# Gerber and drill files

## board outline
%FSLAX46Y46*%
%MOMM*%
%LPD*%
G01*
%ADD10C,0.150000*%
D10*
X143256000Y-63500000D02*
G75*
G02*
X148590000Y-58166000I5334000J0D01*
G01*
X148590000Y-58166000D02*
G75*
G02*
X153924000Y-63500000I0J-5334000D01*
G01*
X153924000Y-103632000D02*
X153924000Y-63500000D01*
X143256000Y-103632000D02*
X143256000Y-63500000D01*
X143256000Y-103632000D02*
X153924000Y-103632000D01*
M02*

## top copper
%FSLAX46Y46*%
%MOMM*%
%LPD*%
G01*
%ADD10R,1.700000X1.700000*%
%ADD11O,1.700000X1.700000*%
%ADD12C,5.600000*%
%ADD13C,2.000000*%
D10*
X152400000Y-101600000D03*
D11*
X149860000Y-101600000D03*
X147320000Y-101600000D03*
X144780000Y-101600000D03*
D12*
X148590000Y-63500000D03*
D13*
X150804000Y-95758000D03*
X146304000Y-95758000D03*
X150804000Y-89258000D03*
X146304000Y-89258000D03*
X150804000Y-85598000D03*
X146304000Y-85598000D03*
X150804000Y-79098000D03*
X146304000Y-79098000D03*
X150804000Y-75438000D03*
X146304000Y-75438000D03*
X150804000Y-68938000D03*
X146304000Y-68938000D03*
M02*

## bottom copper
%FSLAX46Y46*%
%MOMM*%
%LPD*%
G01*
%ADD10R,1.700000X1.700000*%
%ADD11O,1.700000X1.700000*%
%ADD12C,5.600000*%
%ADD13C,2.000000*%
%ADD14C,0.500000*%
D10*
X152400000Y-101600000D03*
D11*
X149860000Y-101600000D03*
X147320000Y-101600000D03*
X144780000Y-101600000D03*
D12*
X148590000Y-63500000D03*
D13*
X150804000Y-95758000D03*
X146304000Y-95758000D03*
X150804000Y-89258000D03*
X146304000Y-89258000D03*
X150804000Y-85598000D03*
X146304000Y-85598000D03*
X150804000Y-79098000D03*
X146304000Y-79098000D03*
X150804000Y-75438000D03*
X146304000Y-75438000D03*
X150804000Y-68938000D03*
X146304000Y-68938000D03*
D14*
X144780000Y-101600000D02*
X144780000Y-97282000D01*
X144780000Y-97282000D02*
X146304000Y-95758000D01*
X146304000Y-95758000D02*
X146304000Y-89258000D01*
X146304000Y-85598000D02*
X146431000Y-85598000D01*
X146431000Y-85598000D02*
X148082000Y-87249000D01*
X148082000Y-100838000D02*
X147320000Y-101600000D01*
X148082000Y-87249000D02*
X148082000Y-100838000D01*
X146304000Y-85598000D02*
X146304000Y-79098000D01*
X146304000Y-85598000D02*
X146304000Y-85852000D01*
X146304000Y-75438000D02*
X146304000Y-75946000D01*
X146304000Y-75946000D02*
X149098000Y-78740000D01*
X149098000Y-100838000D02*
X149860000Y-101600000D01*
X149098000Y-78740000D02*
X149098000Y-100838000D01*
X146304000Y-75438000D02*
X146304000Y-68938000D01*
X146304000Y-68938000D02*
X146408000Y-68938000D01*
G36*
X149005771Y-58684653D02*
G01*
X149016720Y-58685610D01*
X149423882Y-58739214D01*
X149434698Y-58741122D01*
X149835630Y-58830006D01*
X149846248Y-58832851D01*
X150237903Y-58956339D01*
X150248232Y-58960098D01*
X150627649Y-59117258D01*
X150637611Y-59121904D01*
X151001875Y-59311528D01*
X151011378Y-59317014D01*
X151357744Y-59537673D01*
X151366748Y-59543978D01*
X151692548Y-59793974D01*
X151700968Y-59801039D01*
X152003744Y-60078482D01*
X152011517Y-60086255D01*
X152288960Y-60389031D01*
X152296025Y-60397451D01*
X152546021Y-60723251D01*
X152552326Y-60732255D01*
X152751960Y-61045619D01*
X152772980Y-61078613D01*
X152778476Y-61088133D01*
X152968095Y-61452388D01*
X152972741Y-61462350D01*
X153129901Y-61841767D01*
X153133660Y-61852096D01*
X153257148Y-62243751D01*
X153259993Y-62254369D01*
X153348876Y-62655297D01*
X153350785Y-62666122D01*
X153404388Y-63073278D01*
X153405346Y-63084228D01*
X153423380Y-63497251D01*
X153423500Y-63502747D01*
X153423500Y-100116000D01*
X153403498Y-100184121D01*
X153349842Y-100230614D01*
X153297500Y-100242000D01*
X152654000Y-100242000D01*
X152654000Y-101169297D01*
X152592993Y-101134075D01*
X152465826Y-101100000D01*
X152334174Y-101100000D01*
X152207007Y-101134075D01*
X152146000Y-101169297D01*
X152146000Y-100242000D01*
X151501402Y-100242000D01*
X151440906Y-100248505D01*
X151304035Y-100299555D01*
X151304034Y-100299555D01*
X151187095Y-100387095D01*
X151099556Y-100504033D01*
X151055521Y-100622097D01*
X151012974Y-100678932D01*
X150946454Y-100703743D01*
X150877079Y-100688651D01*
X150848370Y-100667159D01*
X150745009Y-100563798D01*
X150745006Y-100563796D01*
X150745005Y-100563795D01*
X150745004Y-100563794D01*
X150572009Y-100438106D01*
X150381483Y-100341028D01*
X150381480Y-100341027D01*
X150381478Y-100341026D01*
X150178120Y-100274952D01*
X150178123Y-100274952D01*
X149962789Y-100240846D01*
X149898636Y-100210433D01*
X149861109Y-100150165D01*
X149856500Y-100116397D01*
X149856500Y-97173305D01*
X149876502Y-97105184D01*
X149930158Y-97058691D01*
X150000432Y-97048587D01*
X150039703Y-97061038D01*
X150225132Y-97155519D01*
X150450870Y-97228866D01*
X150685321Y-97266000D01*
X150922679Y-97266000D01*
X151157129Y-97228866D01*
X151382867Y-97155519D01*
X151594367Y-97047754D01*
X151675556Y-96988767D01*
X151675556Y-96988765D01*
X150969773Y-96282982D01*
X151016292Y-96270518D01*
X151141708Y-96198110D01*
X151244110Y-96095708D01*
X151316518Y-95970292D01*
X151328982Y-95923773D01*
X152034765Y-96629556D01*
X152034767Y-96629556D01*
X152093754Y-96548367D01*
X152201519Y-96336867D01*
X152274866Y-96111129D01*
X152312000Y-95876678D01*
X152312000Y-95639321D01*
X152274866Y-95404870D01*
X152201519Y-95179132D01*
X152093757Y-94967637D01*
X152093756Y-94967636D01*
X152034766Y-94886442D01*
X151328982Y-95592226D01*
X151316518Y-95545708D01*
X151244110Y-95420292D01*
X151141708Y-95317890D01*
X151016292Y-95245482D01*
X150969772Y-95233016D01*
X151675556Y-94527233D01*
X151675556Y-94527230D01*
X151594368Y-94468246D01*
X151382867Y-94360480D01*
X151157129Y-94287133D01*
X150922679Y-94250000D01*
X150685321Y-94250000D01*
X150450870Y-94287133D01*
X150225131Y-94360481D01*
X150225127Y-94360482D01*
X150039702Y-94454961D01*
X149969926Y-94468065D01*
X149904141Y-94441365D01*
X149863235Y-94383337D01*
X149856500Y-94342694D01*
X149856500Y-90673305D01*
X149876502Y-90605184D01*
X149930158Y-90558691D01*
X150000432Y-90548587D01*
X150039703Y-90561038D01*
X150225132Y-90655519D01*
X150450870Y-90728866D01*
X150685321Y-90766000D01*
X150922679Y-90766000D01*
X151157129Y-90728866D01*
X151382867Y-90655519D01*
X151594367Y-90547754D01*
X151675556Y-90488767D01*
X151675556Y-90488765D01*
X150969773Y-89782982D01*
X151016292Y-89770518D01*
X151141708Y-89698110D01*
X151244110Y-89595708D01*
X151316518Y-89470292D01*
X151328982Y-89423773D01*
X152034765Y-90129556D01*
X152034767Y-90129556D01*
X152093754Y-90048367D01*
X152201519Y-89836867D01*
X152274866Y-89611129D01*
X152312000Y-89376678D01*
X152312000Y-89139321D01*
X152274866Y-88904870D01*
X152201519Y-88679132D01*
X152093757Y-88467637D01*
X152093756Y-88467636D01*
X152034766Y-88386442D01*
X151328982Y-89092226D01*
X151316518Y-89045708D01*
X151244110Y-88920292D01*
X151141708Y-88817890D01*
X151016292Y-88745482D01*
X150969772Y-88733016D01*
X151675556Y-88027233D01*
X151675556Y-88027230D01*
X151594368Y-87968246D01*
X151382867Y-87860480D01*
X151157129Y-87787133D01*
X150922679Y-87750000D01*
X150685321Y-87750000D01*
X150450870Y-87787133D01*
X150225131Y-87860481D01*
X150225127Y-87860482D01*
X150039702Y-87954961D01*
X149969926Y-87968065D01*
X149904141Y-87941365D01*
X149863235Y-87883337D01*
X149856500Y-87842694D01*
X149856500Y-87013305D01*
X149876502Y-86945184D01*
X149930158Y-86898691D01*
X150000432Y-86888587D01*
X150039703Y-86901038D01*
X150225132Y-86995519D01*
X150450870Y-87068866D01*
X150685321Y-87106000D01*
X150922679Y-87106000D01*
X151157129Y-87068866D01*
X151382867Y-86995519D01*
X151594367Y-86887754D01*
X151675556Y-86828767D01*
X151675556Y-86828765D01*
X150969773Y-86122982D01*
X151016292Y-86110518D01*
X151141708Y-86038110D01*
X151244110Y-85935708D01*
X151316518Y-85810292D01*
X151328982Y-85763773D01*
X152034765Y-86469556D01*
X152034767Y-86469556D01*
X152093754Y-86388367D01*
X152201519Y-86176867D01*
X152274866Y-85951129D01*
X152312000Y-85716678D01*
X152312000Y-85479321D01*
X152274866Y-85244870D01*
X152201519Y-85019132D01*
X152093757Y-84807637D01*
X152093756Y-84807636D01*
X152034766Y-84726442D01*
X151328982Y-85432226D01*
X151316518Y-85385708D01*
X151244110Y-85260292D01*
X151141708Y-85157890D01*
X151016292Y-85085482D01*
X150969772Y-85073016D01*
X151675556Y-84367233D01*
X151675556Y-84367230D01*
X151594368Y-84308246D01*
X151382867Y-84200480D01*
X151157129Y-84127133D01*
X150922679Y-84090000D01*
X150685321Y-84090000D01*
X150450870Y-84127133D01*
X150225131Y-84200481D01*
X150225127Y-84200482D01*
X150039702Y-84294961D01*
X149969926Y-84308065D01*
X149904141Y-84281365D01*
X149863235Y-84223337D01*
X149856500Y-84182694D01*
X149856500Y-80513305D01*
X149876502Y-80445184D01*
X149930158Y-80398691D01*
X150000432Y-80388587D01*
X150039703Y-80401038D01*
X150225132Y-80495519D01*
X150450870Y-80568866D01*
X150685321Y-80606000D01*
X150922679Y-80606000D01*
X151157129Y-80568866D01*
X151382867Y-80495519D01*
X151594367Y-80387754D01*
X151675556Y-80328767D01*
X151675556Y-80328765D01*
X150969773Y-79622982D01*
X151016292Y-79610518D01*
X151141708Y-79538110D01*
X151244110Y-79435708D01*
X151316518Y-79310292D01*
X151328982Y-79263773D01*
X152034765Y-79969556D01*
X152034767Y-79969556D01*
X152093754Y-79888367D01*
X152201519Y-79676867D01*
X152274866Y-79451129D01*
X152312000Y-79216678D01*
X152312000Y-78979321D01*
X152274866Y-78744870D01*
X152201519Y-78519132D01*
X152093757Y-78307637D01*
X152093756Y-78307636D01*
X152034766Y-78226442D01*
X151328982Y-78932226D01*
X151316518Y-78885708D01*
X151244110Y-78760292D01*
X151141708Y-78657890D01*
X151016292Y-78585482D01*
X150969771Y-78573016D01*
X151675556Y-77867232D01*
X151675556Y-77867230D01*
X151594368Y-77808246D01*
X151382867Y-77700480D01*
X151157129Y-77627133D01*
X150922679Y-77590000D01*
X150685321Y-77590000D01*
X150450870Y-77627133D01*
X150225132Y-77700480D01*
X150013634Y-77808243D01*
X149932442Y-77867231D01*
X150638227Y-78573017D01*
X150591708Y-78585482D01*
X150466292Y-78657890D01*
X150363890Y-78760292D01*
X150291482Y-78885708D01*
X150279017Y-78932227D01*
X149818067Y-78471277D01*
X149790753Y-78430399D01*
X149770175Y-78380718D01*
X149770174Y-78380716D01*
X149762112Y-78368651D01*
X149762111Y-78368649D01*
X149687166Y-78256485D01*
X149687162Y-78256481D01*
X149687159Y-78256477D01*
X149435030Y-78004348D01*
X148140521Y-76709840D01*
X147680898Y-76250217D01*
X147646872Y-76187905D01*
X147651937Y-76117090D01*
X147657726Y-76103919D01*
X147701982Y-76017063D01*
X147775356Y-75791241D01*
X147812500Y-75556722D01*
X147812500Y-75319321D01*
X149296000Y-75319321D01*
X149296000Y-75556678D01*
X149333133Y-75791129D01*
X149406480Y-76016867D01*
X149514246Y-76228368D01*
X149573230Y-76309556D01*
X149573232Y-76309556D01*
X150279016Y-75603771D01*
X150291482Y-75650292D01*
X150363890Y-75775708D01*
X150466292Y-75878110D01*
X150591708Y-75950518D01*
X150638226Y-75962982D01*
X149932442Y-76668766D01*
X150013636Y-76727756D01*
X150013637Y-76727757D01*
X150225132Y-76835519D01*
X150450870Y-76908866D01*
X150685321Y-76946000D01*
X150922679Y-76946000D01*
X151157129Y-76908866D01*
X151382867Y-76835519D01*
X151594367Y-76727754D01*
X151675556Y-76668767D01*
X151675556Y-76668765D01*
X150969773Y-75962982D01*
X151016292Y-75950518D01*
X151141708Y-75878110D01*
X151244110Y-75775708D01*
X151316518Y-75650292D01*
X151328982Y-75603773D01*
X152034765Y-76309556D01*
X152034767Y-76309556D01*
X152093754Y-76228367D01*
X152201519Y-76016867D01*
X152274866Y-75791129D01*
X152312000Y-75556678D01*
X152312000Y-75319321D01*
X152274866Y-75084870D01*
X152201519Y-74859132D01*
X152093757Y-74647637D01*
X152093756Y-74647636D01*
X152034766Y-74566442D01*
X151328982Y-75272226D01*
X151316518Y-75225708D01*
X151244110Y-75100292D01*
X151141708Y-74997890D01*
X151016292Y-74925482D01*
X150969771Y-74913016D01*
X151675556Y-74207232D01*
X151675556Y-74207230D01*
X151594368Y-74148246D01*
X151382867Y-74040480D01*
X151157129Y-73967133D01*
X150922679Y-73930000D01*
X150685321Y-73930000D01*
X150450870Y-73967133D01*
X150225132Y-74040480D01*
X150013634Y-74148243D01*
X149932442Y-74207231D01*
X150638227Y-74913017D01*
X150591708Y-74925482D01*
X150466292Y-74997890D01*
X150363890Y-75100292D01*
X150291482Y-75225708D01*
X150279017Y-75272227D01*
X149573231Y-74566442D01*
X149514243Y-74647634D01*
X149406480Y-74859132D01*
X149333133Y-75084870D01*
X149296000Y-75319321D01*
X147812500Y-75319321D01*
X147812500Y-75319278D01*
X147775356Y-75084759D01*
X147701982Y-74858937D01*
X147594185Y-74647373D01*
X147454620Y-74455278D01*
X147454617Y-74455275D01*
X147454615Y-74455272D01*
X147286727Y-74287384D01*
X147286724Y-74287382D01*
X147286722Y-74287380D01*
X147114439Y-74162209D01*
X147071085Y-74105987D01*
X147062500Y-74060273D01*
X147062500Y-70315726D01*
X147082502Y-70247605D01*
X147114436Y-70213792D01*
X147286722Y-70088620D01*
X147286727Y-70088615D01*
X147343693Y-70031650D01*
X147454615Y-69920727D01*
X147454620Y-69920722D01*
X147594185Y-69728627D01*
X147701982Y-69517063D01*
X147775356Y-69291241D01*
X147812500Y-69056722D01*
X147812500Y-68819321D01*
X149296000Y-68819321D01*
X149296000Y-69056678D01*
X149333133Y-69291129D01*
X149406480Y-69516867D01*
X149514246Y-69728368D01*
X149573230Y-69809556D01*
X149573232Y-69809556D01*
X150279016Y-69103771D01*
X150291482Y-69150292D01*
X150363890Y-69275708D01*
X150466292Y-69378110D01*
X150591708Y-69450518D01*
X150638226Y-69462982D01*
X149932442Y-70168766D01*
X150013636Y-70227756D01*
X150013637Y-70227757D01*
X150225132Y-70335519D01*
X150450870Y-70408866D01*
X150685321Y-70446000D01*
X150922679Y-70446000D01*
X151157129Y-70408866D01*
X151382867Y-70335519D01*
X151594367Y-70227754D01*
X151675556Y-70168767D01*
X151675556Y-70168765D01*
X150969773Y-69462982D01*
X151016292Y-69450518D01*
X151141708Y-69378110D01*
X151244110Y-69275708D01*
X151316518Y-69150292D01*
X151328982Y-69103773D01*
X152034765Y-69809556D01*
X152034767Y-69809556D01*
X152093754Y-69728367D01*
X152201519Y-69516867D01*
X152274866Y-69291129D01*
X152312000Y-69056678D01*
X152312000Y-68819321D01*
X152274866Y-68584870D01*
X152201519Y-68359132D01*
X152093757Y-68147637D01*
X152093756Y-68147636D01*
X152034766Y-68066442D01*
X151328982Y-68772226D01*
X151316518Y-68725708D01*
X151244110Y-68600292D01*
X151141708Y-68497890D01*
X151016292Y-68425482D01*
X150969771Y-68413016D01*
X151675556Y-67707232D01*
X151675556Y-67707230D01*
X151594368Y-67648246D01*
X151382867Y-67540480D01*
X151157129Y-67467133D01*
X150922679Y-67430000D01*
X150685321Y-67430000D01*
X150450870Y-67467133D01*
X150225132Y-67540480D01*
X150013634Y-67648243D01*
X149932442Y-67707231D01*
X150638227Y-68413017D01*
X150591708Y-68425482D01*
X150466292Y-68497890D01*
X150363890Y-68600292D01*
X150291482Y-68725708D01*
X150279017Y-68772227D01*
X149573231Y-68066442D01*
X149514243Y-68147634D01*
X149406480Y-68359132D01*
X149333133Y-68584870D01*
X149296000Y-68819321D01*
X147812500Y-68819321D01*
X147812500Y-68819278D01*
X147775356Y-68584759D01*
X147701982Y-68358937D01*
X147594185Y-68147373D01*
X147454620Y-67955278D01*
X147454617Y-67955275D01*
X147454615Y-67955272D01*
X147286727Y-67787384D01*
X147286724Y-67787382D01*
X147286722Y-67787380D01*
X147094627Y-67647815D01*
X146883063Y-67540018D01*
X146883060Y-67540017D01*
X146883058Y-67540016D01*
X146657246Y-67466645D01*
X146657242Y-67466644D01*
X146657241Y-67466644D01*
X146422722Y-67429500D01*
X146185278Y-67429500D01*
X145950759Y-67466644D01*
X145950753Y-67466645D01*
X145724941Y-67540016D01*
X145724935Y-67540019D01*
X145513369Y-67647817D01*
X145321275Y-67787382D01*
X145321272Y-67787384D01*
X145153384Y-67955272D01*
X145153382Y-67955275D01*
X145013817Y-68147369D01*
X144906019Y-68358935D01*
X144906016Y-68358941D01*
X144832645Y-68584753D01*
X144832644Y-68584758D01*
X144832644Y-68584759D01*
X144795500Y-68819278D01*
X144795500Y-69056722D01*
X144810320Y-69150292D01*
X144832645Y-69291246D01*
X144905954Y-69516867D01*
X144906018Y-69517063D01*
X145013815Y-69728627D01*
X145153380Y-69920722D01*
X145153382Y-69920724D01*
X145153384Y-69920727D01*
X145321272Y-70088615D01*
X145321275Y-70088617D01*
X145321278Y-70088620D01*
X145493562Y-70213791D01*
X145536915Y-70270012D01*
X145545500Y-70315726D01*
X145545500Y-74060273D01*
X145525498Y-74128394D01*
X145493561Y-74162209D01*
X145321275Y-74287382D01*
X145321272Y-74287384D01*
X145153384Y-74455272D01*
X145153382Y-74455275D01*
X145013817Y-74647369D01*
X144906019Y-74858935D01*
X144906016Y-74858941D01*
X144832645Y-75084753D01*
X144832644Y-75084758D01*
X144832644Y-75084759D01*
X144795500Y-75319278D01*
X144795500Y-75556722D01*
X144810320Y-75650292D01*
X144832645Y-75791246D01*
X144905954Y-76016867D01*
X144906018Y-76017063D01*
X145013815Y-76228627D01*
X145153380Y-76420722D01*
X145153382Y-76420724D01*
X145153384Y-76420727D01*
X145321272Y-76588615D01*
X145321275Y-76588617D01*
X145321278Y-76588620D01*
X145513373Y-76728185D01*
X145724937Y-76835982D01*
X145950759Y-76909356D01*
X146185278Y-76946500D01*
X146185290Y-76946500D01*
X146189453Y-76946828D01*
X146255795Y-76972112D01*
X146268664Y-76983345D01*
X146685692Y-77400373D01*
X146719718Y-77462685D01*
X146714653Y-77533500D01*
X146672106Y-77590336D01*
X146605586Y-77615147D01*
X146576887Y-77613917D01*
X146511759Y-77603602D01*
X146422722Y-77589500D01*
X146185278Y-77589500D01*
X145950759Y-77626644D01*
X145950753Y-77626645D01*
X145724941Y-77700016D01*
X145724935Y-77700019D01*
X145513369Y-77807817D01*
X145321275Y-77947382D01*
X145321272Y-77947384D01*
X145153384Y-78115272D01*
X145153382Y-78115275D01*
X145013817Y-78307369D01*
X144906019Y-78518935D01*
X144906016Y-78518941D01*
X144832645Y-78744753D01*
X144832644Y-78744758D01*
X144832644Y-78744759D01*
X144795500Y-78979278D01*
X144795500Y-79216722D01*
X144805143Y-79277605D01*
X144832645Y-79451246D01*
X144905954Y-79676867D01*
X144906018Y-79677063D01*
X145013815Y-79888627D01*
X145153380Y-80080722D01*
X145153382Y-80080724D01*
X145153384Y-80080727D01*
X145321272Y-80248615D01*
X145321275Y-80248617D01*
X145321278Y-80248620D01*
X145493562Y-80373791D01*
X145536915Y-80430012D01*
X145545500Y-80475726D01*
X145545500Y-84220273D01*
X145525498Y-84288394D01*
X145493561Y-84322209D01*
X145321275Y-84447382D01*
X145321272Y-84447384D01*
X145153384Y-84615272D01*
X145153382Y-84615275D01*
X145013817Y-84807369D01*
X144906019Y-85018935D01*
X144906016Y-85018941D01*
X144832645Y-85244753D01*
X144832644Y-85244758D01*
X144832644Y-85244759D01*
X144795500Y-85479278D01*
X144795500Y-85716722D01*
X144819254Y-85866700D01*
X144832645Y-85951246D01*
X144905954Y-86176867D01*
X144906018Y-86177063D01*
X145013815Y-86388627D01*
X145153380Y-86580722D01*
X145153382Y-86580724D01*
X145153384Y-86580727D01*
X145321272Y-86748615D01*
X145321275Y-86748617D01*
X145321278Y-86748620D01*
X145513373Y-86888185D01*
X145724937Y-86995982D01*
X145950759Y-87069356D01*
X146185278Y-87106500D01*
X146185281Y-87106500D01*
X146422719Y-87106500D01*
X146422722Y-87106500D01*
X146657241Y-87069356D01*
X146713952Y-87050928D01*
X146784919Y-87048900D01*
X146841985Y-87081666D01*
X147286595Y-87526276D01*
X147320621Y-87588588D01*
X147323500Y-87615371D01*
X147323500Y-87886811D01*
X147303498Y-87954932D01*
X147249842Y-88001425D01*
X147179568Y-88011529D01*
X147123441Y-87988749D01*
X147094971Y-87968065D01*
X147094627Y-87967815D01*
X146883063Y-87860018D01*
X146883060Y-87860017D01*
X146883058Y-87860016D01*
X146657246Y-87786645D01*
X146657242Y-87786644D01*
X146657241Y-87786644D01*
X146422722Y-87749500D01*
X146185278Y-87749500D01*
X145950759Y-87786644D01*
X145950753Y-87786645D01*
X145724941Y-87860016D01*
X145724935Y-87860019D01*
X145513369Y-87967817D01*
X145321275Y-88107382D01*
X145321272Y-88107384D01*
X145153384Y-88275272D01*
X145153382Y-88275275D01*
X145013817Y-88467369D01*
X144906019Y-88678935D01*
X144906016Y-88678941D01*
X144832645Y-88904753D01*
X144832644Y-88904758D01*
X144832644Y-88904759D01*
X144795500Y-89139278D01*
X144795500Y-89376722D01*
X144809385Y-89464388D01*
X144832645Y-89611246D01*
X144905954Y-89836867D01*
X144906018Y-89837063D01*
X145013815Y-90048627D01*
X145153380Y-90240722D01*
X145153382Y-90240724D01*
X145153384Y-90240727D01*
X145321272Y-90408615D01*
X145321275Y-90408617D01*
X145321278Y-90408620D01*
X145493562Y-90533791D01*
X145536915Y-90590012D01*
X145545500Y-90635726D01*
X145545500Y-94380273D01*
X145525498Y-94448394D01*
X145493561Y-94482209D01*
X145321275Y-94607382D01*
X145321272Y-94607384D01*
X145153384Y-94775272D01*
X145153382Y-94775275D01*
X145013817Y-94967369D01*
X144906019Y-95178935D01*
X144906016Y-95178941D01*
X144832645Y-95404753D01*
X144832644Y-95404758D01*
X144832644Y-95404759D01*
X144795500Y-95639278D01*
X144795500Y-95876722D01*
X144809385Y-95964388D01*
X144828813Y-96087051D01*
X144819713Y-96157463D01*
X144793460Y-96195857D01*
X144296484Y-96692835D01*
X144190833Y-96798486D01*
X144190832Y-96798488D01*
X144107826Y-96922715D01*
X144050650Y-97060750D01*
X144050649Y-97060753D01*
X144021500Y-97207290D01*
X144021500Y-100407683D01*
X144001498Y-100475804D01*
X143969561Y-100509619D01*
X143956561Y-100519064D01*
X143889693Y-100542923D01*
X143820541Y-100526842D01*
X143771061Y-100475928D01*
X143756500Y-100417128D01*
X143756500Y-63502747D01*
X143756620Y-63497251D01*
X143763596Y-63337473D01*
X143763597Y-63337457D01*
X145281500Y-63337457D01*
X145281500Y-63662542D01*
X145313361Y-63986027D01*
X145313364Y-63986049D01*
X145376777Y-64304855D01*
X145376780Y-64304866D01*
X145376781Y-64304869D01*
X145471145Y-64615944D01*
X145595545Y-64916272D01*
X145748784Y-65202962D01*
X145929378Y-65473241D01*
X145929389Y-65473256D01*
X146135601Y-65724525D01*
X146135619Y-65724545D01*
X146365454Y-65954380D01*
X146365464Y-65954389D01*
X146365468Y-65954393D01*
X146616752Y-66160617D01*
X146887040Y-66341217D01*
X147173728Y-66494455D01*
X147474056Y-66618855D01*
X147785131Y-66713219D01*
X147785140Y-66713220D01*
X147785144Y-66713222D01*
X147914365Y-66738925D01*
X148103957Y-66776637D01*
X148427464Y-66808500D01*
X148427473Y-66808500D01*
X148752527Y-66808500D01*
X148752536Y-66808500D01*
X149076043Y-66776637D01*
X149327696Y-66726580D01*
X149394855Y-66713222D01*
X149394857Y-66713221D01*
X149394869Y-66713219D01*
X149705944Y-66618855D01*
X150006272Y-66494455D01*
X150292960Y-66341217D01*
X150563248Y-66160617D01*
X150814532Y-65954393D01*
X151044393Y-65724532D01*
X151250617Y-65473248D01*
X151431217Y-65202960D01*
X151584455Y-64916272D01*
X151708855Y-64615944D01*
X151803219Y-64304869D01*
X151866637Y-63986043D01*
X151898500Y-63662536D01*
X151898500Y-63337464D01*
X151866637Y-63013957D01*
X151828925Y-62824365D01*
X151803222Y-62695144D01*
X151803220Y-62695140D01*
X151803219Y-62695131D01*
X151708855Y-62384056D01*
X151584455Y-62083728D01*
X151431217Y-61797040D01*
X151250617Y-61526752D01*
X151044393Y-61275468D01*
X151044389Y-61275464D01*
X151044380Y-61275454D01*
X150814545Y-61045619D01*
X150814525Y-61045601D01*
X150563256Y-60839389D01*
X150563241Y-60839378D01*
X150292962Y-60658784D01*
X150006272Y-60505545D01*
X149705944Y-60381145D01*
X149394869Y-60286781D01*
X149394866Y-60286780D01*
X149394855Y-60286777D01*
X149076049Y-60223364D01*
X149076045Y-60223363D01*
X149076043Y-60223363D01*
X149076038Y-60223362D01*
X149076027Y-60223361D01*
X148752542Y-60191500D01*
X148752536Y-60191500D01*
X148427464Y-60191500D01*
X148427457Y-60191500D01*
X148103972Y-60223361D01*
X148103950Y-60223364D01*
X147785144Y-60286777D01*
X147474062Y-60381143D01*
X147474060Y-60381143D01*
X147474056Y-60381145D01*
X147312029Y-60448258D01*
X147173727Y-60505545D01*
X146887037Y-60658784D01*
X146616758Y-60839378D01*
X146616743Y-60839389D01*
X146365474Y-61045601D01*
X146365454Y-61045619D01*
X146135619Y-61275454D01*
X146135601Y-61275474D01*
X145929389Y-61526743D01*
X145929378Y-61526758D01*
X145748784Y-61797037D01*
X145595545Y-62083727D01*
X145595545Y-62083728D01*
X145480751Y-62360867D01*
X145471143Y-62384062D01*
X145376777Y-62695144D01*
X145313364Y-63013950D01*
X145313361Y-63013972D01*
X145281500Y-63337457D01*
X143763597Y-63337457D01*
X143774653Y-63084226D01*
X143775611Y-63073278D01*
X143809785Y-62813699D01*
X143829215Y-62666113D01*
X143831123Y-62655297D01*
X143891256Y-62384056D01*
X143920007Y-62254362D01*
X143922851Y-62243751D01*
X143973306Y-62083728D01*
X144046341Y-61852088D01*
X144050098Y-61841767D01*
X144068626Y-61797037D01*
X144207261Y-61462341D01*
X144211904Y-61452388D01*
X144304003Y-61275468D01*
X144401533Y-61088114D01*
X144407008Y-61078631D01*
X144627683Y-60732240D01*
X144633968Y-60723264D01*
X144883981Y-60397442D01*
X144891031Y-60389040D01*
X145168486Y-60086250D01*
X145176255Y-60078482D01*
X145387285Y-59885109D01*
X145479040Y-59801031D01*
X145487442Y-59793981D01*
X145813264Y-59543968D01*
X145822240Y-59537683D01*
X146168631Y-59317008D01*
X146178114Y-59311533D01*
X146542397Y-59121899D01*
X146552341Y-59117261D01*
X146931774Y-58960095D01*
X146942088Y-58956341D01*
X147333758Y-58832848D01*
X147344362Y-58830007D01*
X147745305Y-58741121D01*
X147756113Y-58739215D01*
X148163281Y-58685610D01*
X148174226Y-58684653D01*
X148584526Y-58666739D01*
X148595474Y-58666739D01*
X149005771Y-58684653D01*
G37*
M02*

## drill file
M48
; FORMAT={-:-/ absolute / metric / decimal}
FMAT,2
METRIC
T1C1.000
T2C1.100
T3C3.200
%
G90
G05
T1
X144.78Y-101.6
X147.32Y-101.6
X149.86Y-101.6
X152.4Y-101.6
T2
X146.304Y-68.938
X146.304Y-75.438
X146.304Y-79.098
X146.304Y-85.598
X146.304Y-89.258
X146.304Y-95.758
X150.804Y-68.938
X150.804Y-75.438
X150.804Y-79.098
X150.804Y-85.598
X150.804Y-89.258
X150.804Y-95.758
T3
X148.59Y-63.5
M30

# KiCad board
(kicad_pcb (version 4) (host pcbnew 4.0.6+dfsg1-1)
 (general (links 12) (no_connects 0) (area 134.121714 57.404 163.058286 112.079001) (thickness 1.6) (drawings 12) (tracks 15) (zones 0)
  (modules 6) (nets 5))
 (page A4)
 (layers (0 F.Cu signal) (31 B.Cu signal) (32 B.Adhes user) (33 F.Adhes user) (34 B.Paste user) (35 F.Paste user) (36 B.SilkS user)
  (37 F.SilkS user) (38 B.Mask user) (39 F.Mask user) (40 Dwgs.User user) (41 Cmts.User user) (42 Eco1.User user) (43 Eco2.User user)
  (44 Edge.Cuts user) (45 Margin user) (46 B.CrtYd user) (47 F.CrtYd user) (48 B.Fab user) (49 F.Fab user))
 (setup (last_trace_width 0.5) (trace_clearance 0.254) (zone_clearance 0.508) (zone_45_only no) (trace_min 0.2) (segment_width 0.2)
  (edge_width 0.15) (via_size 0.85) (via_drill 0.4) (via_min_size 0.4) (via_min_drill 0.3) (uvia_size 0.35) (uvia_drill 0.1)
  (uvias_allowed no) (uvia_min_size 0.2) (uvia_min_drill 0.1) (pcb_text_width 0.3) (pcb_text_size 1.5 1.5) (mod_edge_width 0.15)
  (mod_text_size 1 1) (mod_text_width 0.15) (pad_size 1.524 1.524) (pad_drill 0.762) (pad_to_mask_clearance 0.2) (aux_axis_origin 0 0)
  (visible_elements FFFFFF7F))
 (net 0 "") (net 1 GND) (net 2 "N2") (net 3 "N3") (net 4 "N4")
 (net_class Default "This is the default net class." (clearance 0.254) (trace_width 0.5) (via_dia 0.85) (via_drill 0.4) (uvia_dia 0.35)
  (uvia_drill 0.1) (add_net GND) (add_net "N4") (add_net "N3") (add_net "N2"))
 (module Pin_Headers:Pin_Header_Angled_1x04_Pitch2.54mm (layer F.Cu) (at 152.4 101.6 270)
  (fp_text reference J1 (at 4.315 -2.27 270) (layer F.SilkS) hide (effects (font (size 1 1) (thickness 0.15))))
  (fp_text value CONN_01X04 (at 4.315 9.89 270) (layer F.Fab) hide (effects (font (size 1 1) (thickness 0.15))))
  (pad 1 thru_hole rect (at 0 0 270) (size 1.7 1.7) (drill 1) (layers *.Cu *.Mask) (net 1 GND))
  (pad 2 thru_hole oval (at 0 2.54 270) (size 1.7 1.7) (drill 1) (layers *.Cu *.Mask) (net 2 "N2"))
  (pad 3 thru_hole oval (at 0 5.08 270) (size 1.7 1.7) (drill 1) (layers *.Cu *.Mask) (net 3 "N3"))
  (pad 4 thru_hole oval (at 0 7.62 270) (size 1.7 1.7) (drill 1) (layers *.Cu *.Mask) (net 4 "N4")))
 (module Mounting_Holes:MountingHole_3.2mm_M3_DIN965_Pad (layer F.Cu) (at 148.59 63.5)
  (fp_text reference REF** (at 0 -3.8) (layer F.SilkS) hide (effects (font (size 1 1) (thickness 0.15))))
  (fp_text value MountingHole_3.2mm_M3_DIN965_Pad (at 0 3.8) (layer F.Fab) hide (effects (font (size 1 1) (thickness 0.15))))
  (pad 1 thru_hole circle (at 0 0) (size 5.6 5.6) (drill 3.2) (layers *.Cu *.Mask)))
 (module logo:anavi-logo (layer F.Cu) (at 144.272 87.757 90)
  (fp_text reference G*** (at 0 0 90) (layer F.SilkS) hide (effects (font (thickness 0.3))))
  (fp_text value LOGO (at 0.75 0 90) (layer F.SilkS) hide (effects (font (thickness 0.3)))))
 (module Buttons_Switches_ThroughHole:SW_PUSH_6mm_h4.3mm (layer F.Cu) (at 146.304 95.758 90)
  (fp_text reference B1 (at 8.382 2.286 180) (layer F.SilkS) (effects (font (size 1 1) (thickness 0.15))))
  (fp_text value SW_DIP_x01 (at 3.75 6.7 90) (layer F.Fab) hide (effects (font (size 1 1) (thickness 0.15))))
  (pad 2 thru_hole circle (at 0 4.5 180) (size 2 2) (drill 1.1) (layers *.Cu *.Mask) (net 1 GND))
  (pad 1 thru_hole circle (at 0 0 180) (size 2 2) (drill 1.1) (layers *.Cu *.Mask) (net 4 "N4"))
  (pad 2 thru_hole circle (at 6.5 4.5 180) (size 2 2) (drill 1.1) (layers *.Cu *.Mask) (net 1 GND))
  (pad 1 thru_hole circle (at 6.5 0 180) (size 2 2) (drill 1.1) (layers *.Cu *.Mask) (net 4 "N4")))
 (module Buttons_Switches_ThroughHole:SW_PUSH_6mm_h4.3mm (layer F.Cu) (at 146.304 85.598 90)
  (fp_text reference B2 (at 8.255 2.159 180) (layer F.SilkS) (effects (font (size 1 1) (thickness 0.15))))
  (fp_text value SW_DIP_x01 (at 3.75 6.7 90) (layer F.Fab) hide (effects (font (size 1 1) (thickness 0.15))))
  (pad 2 thru_hole circle (at 0 4.5 180) (size 2 2) (drill 1.1) (layers *.Cu *.Mask) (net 1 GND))
  (pad 1 thru_hole circle (at 0 0 180) (size 2 2) (drill 1.1) (layers *.Cu *.Mask) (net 3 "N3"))
  (pad 2 thru_hole circle (at 6.5 4.5 180) (size 2 2) (drill 1.1) (layers *.Cu *.Mask) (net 1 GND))
  (pad 1 thru_hole circle (at 6.5 0 180) (size 2 2) (drill 1.1) (layers *.Cu *.Mask) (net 3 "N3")))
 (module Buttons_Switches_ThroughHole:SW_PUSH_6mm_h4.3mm (layer F.Cu) (at 146.304 75.438 90)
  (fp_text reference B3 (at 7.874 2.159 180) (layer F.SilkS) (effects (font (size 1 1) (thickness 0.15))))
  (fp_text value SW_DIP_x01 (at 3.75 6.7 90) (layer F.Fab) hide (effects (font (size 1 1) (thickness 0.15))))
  (pad 2 thru_hole circle (at 0 4.5 180) (size 2 2) (drill 1.1) (layers *.Cu *.Mask) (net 1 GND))
  (pad 1 thru_hole circle (at 0 0 180) (size 2 2) (drill 1.1) (layers *.Cu *.Mask) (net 2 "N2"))
  (pad 2 thru_hole circle (at 6.5 4.5 180) (size 2 2) (drill 1.1) (layers *.Cu *.Mask) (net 1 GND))
  (pad 1 thru_hole circle (at 6.5 0 180) (size 2 2) (drill 1.1) (layers *.Cu *.Mask) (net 2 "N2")))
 (gr_arc (start 148.59 63.5) (end 143.256 63.5) (angle 90) (layer Edge.Cuts) (width 0.15))
 (gr_arc (start 148.59 63.5) (end 148.59 58.166) (angle 90) (layer Edge.Cuts) (width 0.15))
 (gr_line (start 153.924 103.632) (end 153.924 63.5) (angle 90) (layer Edge.Cuts) (width 0.15))
 (gr_line (start 143.256 103.632) (end 143.256 63.5) (angle 90) (layer Edge.Cuts) (width 0.15))
 (gr_line (start 143.256 103.632) (end 153.924 103.632) (angle 90) (layer Edge.Cuts) (width 0.15))
 (segment (start 144.78 101.6) (end 144.78 97.282) (width 0.5) (layer B.Cu) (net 4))
 (segment (start 144.78 97.282) (end 146.304 95.758) (width 0.5) (layer B.Cu) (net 4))
 (segment (start 146.304 95.758) (end 146.304 89.258) (width 0.5) (layer B.Cu) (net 4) (status 30))
 (segment (start 146.304 85.598) (end 146.431 85.598) (width 0.5) (layer B.Cu) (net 3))
 (segment (start 146.431 85.598) (end 148.082 87.249) (width 0.5) (layer B.Cu) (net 3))
 (segment (start 148.082 100.838) (end 147.32 101.6) (width 0.5) (layer B.Cu) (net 3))
 (segment (start 148.082 87.249) (end 148.082 100.838) (width 0.5) (layer B.Cu) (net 3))
 (segment (start 146.304 85.598) (end 146.304 79.098) (width 0.5) (layer B.Cu) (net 3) (status 30))
 (segment (start 146.304 85.598) (end 146.304 85.852) (width 0.5) (layer B.Cu) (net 3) (status 30))
 (segment (start 146.304 75.438) (end 146.304 75.946) (width 0.5) (layer B.Cu) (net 2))
 (segment (start 146.304 75.946) (end 149.098 78.74) (width 0.5) (layer B.Cu) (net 2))
 (segment (start 149.098 100.838) (end 149.86 101.6) (width 0.5) (layer B.Cu) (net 2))
 (segment (start 149.098 78.74) (end 149.098 100.838) (width 0.5) (layer B.Cu) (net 2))
 (segment (start 146.304 75.438) (end 146.304 68.938) (width 0.5) (layer B.Cu) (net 2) (status 30))
 (segment (start 146.304 68.938) (end 146.408 68.938) (width 0.5) (layer B.Cu) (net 2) (status 30))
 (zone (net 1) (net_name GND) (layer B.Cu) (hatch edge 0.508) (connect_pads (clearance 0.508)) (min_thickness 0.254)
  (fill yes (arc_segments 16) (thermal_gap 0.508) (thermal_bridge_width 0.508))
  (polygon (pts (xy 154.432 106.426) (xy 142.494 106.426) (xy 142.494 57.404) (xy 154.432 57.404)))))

